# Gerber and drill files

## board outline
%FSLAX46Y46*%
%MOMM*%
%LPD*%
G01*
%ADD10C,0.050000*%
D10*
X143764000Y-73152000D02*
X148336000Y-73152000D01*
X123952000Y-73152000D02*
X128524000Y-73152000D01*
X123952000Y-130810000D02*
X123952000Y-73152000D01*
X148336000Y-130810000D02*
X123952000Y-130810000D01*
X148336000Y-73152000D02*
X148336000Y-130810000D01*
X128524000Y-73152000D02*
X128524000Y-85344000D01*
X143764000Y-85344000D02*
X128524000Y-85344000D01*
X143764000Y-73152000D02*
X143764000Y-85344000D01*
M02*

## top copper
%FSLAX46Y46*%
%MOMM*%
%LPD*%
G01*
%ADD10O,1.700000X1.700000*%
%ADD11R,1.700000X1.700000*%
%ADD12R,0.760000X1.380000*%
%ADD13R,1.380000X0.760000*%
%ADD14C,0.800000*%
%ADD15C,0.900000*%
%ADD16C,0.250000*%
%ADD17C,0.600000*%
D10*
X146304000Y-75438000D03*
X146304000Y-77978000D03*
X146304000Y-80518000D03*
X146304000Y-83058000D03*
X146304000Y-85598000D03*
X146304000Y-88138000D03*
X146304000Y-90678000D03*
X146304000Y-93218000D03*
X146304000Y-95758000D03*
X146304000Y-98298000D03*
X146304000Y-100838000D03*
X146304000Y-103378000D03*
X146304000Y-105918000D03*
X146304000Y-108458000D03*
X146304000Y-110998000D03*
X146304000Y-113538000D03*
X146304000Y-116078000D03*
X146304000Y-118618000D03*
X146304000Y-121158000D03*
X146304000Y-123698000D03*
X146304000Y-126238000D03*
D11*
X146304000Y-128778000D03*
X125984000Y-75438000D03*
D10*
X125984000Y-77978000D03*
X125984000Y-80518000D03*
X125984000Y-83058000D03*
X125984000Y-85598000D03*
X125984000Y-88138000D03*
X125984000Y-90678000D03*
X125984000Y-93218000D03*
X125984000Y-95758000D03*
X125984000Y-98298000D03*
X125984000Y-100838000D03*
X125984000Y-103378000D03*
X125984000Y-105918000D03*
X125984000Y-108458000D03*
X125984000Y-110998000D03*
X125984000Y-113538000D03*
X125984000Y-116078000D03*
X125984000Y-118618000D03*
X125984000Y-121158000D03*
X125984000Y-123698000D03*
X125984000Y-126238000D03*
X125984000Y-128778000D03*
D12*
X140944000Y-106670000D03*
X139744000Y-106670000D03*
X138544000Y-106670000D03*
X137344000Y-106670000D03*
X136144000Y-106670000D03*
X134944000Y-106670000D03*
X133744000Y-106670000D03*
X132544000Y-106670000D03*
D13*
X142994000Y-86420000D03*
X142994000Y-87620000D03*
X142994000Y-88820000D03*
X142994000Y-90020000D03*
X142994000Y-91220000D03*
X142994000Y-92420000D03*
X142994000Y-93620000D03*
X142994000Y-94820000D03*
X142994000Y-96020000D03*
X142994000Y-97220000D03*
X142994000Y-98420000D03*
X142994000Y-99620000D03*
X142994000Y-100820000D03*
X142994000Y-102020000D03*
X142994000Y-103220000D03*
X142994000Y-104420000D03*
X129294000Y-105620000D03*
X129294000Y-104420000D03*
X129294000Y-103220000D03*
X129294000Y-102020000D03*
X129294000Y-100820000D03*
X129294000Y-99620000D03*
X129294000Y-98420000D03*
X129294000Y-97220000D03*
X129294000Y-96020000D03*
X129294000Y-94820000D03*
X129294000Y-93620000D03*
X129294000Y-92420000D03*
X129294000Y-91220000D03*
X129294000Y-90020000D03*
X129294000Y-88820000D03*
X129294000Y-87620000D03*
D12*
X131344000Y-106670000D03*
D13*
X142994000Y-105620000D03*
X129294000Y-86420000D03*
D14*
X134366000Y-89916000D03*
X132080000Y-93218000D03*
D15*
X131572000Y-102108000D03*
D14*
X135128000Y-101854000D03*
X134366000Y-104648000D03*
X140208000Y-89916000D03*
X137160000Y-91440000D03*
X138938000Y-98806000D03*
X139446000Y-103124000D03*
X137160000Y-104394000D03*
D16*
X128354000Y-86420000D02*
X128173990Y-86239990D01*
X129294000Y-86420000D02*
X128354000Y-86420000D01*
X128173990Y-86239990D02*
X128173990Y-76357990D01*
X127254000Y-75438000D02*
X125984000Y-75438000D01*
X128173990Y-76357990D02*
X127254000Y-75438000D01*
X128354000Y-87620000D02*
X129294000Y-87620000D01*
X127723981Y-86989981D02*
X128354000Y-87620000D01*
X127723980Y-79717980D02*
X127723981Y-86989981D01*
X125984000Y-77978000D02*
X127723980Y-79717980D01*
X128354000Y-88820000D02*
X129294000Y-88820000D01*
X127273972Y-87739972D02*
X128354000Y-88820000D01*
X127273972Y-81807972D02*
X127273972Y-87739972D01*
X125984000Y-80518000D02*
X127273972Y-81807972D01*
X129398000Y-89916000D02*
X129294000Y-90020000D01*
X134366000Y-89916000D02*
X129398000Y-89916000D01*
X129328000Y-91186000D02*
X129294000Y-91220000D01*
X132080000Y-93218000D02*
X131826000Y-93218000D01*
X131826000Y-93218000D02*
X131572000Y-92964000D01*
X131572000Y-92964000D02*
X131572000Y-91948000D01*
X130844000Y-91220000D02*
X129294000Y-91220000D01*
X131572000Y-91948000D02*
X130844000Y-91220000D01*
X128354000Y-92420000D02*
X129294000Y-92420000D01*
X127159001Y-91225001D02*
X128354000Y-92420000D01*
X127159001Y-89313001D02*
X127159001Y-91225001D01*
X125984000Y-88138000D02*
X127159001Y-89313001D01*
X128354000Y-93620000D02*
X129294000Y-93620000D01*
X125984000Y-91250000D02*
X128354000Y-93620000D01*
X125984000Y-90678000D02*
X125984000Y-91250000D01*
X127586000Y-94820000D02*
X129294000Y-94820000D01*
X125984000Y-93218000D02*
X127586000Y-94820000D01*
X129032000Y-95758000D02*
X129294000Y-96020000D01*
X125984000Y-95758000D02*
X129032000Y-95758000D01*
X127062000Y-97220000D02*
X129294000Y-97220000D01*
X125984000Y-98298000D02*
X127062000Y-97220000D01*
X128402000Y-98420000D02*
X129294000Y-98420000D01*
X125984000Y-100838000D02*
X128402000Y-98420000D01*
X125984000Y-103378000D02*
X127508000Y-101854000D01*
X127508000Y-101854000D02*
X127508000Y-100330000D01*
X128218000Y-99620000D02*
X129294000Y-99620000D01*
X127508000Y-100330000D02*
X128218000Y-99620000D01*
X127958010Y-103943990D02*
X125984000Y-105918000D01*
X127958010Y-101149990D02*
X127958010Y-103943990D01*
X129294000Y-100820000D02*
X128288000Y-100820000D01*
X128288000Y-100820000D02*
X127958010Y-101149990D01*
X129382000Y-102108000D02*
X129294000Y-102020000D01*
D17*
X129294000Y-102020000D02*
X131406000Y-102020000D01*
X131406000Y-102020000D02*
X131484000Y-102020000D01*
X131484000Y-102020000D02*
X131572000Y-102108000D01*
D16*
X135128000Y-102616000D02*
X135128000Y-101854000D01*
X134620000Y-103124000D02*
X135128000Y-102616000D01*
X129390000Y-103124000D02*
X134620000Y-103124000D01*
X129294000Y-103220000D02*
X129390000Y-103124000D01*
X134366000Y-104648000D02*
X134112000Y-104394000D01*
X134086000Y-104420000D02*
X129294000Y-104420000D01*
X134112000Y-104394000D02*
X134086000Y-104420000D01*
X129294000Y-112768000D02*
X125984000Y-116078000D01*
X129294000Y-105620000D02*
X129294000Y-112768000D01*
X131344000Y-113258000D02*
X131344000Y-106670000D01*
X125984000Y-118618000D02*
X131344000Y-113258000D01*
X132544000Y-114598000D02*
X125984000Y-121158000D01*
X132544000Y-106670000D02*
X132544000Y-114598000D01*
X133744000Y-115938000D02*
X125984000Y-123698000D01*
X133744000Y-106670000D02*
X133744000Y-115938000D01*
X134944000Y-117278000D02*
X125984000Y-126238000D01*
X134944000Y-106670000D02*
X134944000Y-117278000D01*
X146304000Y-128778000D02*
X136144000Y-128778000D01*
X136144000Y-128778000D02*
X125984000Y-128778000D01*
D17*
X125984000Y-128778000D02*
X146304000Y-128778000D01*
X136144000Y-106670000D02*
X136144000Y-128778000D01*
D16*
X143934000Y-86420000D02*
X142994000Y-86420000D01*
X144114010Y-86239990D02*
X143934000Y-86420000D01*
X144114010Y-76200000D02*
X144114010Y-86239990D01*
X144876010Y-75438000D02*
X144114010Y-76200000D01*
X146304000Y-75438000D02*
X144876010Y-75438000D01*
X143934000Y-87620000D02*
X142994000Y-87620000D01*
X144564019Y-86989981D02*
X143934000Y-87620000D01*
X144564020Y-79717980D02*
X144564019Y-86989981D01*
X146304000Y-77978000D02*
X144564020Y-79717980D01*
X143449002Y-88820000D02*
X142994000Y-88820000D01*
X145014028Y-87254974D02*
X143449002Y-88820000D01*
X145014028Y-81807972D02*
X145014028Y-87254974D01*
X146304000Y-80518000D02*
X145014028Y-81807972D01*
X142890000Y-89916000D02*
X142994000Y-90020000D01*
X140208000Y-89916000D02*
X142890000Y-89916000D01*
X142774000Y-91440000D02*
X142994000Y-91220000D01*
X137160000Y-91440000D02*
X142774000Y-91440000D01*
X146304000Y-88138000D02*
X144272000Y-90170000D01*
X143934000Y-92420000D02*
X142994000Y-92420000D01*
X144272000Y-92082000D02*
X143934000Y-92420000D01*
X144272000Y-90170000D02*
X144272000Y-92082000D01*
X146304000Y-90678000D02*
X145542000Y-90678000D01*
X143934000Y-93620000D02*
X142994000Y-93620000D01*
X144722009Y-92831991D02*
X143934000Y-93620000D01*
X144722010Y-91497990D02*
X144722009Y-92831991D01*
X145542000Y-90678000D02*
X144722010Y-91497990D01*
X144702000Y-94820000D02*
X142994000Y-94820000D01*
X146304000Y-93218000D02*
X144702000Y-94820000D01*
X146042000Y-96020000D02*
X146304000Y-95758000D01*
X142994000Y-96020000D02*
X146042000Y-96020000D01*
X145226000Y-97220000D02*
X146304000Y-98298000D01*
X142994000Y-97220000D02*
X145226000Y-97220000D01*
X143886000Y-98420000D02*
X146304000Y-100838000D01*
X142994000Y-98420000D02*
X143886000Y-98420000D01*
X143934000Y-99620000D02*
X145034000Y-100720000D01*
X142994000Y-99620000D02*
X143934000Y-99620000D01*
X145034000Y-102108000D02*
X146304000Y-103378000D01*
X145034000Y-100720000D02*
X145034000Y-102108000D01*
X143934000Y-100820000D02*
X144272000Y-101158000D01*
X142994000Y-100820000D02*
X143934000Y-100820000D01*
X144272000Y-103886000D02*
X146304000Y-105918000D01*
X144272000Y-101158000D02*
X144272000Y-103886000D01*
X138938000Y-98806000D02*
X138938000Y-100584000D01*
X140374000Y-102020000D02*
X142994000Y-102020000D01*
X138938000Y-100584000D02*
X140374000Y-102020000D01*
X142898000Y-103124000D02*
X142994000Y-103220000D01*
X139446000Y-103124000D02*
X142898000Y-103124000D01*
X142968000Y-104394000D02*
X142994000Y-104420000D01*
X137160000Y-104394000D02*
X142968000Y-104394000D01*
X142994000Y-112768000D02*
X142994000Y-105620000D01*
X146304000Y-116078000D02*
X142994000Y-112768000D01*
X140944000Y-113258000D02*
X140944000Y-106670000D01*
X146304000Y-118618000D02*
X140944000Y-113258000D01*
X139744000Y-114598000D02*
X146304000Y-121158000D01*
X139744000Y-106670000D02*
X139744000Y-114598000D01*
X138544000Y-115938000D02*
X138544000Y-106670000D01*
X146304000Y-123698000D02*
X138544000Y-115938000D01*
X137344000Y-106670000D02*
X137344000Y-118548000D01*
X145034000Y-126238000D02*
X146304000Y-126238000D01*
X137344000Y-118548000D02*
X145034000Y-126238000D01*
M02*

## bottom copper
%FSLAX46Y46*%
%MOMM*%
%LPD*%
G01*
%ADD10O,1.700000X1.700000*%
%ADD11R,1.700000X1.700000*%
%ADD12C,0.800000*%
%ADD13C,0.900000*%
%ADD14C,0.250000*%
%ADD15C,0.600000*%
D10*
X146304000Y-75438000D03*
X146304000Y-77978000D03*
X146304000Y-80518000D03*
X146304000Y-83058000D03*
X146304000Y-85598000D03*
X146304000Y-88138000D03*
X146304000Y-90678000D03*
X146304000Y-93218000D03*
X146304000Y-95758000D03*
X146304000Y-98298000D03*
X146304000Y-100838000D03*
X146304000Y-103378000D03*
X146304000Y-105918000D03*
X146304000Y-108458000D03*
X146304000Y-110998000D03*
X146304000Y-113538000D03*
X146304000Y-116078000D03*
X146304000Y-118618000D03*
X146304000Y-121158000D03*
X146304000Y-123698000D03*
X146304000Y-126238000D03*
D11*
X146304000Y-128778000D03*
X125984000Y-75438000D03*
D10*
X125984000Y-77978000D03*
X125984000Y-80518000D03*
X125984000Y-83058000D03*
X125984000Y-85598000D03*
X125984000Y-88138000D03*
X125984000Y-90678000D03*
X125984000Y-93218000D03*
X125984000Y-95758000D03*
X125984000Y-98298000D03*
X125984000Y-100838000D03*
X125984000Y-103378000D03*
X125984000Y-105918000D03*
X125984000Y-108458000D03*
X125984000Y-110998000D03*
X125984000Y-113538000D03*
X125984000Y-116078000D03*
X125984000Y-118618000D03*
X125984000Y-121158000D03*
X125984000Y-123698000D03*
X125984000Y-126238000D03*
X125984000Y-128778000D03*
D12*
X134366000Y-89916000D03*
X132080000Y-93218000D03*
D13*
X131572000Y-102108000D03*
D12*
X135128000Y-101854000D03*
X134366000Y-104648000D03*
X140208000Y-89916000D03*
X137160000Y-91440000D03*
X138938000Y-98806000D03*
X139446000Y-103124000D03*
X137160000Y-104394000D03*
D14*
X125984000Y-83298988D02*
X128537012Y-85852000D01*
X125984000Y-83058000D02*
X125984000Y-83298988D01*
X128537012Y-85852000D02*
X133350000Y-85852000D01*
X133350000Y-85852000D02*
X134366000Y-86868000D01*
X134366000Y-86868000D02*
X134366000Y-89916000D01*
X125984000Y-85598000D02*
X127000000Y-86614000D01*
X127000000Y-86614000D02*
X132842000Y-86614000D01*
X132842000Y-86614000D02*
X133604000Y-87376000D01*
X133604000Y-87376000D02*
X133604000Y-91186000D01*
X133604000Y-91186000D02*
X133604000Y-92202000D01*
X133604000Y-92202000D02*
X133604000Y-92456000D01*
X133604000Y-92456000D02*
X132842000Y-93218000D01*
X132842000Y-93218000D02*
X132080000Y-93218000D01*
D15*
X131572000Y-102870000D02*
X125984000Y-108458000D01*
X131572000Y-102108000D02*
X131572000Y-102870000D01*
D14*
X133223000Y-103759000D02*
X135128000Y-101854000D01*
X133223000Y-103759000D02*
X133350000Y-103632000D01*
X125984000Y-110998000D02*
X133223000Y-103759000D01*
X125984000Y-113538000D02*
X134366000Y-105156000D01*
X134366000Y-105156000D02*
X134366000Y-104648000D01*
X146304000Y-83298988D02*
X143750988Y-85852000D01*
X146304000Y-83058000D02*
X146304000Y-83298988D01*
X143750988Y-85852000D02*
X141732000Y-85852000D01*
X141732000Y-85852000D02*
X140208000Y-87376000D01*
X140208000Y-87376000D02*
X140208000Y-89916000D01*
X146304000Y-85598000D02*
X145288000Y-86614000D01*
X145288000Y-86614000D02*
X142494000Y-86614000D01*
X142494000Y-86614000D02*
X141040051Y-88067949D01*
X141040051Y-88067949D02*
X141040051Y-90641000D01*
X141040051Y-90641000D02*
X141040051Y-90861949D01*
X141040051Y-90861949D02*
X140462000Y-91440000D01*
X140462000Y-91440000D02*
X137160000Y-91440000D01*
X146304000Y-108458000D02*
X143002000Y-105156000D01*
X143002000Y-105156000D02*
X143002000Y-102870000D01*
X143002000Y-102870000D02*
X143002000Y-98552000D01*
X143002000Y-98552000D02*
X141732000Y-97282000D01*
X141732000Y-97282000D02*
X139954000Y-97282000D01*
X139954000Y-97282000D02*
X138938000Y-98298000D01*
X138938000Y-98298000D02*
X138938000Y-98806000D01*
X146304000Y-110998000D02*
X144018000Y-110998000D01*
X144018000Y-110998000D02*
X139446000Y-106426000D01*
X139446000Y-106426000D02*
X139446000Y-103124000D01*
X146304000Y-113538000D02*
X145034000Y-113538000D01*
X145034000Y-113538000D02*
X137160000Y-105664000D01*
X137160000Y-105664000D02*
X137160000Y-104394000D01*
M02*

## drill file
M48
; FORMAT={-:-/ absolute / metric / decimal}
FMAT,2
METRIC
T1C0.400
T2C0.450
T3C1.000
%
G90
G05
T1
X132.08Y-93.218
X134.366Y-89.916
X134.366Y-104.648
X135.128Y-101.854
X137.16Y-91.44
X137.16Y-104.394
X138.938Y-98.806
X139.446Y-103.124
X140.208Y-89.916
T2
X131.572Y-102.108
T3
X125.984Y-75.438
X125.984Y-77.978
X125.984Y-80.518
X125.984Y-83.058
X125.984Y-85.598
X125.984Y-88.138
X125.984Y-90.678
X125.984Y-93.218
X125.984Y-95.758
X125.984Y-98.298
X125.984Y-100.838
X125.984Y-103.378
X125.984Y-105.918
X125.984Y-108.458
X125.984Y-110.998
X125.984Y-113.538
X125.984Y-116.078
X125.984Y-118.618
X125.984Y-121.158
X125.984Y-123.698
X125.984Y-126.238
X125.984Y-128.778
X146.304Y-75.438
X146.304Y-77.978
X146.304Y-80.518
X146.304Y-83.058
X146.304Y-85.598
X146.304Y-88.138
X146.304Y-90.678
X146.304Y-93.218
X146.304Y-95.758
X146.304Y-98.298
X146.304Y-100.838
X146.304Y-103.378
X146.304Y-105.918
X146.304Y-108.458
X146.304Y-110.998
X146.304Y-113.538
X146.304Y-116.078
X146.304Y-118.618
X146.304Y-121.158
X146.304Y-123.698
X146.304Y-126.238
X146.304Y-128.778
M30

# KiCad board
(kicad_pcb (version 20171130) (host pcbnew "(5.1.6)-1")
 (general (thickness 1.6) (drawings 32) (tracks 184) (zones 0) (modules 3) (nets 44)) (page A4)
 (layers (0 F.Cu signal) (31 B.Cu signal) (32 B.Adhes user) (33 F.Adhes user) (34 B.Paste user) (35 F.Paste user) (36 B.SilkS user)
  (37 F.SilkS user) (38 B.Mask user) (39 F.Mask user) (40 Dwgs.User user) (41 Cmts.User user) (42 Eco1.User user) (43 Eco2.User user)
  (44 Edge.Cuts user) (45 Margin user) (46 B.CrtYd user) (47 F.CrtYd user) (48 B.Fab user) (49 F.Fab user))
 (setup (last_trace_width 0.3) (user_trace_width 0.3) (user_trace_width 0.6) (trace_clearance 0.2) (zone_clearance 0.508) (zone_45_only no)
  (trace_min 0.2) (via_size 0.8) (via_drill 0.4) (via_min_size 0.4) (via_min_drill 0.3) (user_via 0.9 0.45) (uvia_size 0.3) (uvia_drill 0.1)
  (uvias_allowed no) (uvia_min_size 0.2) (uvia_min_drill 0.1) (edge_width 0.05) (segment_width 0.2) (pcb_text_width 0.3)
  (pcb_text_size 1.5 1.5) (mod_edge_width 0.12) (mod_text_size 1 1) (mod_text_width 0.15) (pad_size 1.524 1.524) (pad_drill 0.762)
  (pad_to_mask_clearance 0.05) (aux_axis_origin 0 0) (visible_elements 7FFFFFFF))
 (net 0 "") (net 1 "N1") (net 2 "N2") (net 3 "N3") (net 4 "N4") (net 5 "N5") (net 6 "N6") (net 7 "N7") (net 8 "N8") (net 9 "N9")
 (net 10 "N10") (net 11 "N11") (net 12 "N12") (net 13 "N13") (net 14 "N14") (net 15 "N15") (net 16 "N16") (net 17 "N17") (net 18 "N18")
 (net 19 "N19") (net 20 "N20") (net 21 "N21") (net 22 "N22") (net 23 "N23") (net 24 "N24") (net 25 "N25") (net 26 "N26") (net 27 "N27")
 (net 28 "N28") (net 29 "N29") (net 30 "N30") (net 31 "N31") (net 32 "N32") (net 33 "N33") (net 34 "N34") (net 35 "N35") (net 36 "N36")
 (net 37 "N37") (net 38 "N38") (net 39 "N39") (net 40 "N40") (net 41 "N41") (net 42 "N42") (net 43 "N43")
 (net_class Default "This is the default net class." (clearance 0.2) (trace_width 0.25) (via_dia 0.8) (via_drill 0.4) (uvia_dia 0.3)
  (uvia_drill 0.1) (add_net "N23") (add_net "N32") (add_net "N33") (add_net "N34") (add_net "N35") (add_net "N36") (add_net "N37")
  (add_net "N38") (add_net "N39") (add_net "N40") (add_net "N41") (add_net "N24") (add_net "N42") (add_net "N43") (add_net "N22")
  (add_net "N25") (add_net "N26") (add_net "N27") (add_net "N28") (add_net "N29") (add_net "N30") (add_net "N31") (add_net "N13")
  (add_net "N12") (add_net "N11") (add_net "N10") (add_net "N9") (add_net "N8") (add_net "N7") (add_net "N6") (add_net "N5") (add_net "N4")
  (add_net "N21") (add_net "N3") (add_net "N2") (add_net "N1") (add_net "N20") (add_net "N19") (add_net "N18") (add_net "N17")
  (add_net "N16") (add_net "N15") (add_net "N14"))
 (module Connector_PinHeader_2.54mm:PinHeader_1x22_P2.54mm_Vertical (layer F.Cu) (at 146.304 128.778 180)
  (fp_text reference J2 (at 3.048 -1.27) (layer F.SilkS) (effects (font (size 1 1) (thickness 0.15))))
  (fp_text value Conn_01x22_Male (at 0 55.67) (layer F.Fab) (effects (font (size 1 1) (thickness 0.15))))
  (pad 22 thru_hole oval (at 0 53.34 180) (size 1.7 1.7) (drill 1) (layers *.Cu *.Mask) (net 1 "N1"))
  (pad 21 thru_hole oval (at 0 50.8 180) (size 1.7 1.7) (drill 1) (layers *.Cu *.Mask) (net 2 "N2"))
  (pad 20 thru_hole oval (at 0 48.26 180) (size 1.7 1.7) (drill 1) (layers *.Cu *.Mask) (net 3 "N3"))
  (pad 19 thru_hole oval (at 0 45.72 180) (size 1.7 1.7) (drill 1) (layers *.Cu *.Mask) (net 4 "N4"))
  (pad 18 thru_hole oval (at 0 43.18 180) (size 1.7 1.7) (drill 1) (layers *.Cu *.Mask) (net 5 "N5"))
  (pad 17 thru_hole oval (at 0 40.64 180) (size 1.7 1.7) (drill 1) (layers *.Cu *.Mask) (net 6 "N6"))
  (pad 16 thru_hole oval (at 0 38.1 180) (size 1.7 1.7) (drill 1) (layers *.Cu *.Mask) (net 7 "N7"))
  (pad 15 thru_hole oval (at 0 35.56 180) (size 1.7 1.7) (drill 1) (layers *.Cu *.Mask) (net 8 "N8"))
  (pad 14 thru_hole oval (at 0 33.02 180) (size 1.7 1.7) (drill 1) (layers *.Cu *.Mask) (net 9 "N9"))
  (pad 13 thru_hole oval (at 0 30.48 180) (size 1.7 1.7) (drill 1) (layers *.Cu *.Mask) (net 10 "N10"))
  (pad 12 thru_hole oval (at 0 27.94 180) (size 1.7 1.7) (drill 1) (layers *.Cu *.Mask) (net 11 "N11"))
  (pad 11 thru_hole oval (at 0 25.4 180) (size 1.7 1.7) (drill 1) (layers *.Cu *.Mask) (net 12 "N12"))
  (pad 10 thru_hole oval (at 0 22.86 180) (size 1.7 1.7) (drill 1) (layers *.Cu *.Mask) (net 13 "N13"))
  (pad 9 thru_hole oval (at 0 20.32 180) (size 1.7 1.7) (drill 1) (layers *.Cu *.Mask) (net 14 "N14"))
  (pad 8 thru_hole oval (at 0 17.78 180) (size 1.7 1.7) (drill 1) (layers *.Cu *.Mask) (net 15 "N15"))
  (pad 7 thru_hole oval (at 0 15.24 180) (size 1.7 1.7) (drill 1) (layers *.Cu *.Mask) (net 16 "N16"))
  (pad 6 thru_hole oval (at 0 12.7 180) (size 1.7 1.7) (drill 1) (layers *.Cu *.Mask) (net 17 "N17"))
  (pad 5 thru_hole oval (at 0 10.16 180) (size 1.7 1.7) (drill 1) (layers *.Cu *.Mask) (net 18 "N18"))
  (pad 4 thru_hole oval (at 0 7.62 180) (size 1.7 1.7) (drill 1) (layers *.Cu *.Mask) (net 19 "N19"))
  (pad 3 thru_hole oval (at 0 5.08 180) (size 1.7 1.7) (drill 1) (layers *.Cu *.Mask) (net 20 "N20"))
  (pad 2 thru_hole oval (at 0 2.54 180) (size 1.7 1.7) (drill 1) (layers *.Cu *.Mask) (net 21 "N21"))
  (pad 1 thru_hole rect (at 0 0 180) (size 1.7 1.7) (drill 1) (layers *.Cu *.Mask) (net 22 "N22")))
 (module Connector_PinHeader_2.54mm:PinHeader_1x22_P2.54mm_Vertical (layer F.Cu) (at 125.984 75.438)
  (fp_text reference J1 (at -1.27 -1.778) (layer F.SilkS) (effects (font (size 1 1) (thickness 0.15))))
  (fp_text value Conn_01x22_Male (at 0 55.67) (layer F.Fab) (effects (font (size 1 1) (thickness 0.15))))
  (pad 1 thru_hole rect (at 0 0) (size 1.7 1.7) (drill 1) (layers *.Cu *.Mask) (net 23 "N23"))
  (pad 2 thru_hole oval (at 0 2.54) (size 1.7 1.7) (drill 1) (layers *.Cu *.Mask) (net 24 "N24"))
  (pad 3 thru_hole oval (at 0 5.08) (size 1.7 1.7) (drill 1) (layers *.Cu *.Mask) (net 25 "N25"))
  (pad 4 thru_hole oval (at 0 7.62) (size 1.7 1.7) (drill 1) (layers *.Cu *.Mask) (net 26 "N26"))
  (pad 5 thru_hole oval (at 0 10.16) (size 1.7 1.7) (drill 1) (layers *.Cu *.Mask) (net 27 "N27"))
  (pad 6 thru_hole oval (at 0 12.7) (size 1.7 1.7) (drill 1) (layers *.Cu *.Mask) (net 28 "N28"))
  (pad 7 thru_hole oval (at 0 15.24) (size 1.7 1.7) (drill 1) (layers *.Cu *.Mask) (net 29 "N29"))
  (pad 8 thru_hole oval (at 0 17.78) (size 1.7 1.7) (drill 1) (layers *.Cu *.Mask) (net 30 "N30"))
  (pad 9 thru_hole oval (at 0 20.32) (size 1.7 1.7) (drill 1) (layers *.Cu *.Mask) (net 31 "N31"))
  (pad 10 thru_hole oval (at 0 22.86) (size 1.7 1.7) (drill 1) (layers *.Cu *.Mask) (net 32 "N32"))
  (pad 11 thru_hole oval (at 0 25.4) (size 1.7 1.7) (drill 1) (layers *.Cu *.Mask) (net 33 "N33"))
  (pad 12 thru_hole oval (at 0 27.94) (size 1.7 1.7) (drill 1) (layers *.Cu *.Mask) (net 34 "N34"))
  (pad 13 thru_hole oval (at 0 30.48) (size 1.7 1.7) (drill 1) (layers *.Cu *.Mask) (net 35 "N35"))
  (pad 14 thru_hole oval (at 0 33.02) (size 1.7 1.7) (drill 1) (layers *.Cu *.Mask) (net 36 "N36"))
  (pad 15 thru_hole oval (at 0 35.56) (size 1.7 1.7) (drill 1) (layers *.Cu *.Mask) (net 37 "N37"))
  (pad 16 thru_hole oval (at 0 38.1) (size 1.7 1.7) (drill 1) (layers *.Cu *.Mask) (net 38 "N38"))
  (pad 17 thru_hole oval (at 0 40.64) (size 1.7 1.7) (drill 1) (layers *.Cu *.Mask) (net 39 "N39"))
  (pad 18 thru_hole oval (at 0 43.18) (size 1.7 1.7) (drill 1) (layers *.Cu *.Mask) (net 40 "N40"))
  (pad 19 thru_hole oval (at 0 45.72) (size 1.7 1.7) (drill 1) (layers *.Cu *.Mask) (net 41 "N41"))
  (pad 20 thru_hole oval (at 0 48.26) (size 1.7 1.7) (drill 1) (layers *.Cu *.Mask) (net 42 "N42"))
  (pad 21 thru_hole oval (at 0 50.8) (size 1.7 1.7) (drill 1) (layers *.Cu *.Mask) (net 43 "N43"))
  (pad 22 thru_hole oval (at 0 53.34) (size 1.7 1.7) (drill 1) (layers *.Cu *.Mask) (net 22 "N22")))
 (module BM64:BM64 (layer F.Cu) (at 136.144 83.82)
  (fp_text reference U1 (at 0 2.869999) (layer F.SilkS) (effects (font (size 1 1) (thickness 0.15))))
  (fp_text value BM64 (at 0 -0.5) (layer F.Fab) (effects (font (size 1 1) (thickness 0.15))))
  (pad 26 smd rect (at 4.8 22.85 90) (size 1.38 0.76) (layers F.Cu F.Paste F.Mask) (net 18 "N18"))
  (pad 25 smd rect (at 3.6 22.85 90) (size 1.38 0.76) (layers F.Cu F.Paste F.Mask) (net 19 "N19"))
  (pad 24 smd rect (at 2.4 22.85 90) (size 1.38 0.76) (layers F.Cu F.Paste F.Mask) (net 20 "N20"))
  (pad 23 smd rect (at 1.2 22.85 90) (size 1.38 0.76) (layers F.Cu F.Paste F.Mask) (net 21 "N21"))
  (pad 22 smd rect (at 0 22.85 90) (size 1.38 0.76) (layers F.Cu F.Paste F.Mask) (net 22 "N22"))
  (pad 21 smd rect (at -1.2 22.85 90) (size 1.38 0.76) (layers F.Cu F.Paste F.Mask) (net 43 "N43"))
  (pad 20 smd rect (at -2.4 22.85 90) (size 1.38 0.76) (layers F.Cu F.Paste F.Mask) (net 42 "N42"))
  (pad 19 smd rect (at -3.6 22.85 90) (size 1.38 0.76) (layers F.Cu F.Paste F.Mask) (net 41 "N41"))
  (pad 43 smd rect (at 6.85 2.6) (size 1.38 0.76) (layers F.Cu F.Paste F.Mask) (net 1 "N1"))
  (pad 42 smd rect (at 6.85 3.8) (size 1.38 0.76) (layers F.Cu F.Paste F.Mask) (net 2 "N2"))
  (pad 41 smd rect (at 6.85 5) (size 1.38 0.76) (layers F.Cu F.Paste F.Mask) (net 3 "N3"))
  (pad 40 smd rect (at 6.85 6.2) (size 1.38 0.76) (layers F.Cu F.Paste F.Mask) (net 4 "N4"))
  (pad 39 smd rect (at 6.85 7.4) (size 1.38 0.76) (layers F.Cu F.Paste F.Mask) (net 5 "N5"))
  (pad 38 smd rect (at 6.85 8.6) (size 1.38 0.76) (layers F.Cu F.Paste F.Mask) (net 6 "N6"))
  (pad 37 smd rect (at 6.85 9.8) (size 1.38 0.76) (layers F.Cu F.Paste F.Mask) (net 7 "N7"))
  (pad 36 smd rect (at 6.85 11) (size 1.38 0.76) (layers F.Cu F.Paste F.Mask) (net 8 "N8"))
  (pad 35 smd rect (at 6.85 12.2) (size 1.38 0.76) (layers F.Cu F.Paste F.Mask) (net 9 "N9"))
  (pad 34 smd rect (at 6.85 13.4) (size 1.38 0.76) (layers F.Cu F.Paste F.Mask) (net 10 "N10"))
  (pad 33 smd rect (at 6.85 14.6) (size 1.38 0.76) (layers F.Cu F.Paste F.Mask) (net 11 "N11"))
  (pad 32 smd rect (at 6.85 15.8) (size 1.38 0.76) (layers F.Cu F.Paste F.Mask) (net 12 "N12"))
  (pad 31 smd rect (at 6.85 17) (size 1.38 0.76) (layers F.Cu F.Paste F.Mask) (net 13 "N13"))
  (pad 30 smd rect (at 6.85 18.2) (size 1.38 0.76) (layers F.Cu F.Paste F.Mask) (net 14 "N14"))
  (pad 29 smd rect (at 6.85 19.4) (size 1.38 0.76) (layers F.Cu F.Paste F.Mask) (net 15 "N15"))
  (pad 28 smd rect (at 6.85 20.6) (size 1.38 0.76) (layers F.Cu F.Paste F.Mask) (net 16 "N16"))
  (pad 17 smd rect (at -6.85 21.8) (size 1.38 0.76) (layers F.Cu F.Paste F.Mask) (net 39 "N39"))
  (pad 16 smd rect (at -6.85 20.6) (size 1.38 0.76) (layers F.Cu F.Paste F.Mask) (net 38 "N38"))
  (pad 15 smd rect (at -6.85 19.4) (size 1.38 0.76) (layers F.Cu F.Paste F.Mask) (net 37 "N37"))
  (pad 14 smd rect (at -6.85 18.2) (size 1.38 0.76) (layers F.Cu F.Paste F.Mask) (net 36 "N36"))
  (pad 13 smd rect (at -6.85 17) (size 1.38 0.76) (layers F.Cu F.Paste F.Mask) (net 35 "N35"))
  (pad 12 smd rect (at -6.85 15.8) (size 1.38 0.76) (layers F.Cu F.Paste F.Mask) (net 34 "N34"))
  (pad 11 smd rect (at -6.85 14.6) (size 1.38 0.76) (layers F.Cu F.Paste F.Mask) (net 33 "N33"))
  (pad 10 smd rect (at -6.85 13.4) (size 1.38 0.76) (layers F.Cu F.Paste F.Mask) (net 32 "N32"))
  (pad 9 smd rect (at -6.85 12.2) (size 1.38 0.76) (layers F.Cu F.Paste F.Mask) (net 31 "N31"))
  (pad 8 smd rect (at -6.85 11) (size 1.38 0.76) (layers F.Cu F.Paste F.Mask) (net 30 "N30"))
  (pad 7 smd rect (at -6.85 9.8) (size 1.38 0.76) (layers F.Cu F.Paste F.Mask) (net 29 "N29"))
  (pad 6 smd rect (at -6.85 8.6) (size 1.38 0.76) (layers F.Cu F.Paste F.Mask) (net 28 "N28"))
  (pad 5 smd rect (at -6.85 7.4) (size 1.38 0.76) (layers F.Cu F.Paste F.Mask) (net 27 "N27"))
  (pad 4 smd rect (at -6.85 6.2) (size 1.38 0.76) (layers F.Cu F.Paste F.Mask) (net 26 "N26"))
  (pad 3 smd rect (at -6.85 5) (size 1.38 0.76) (layers F.Cu F.Paste F.Mask) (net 25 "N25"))
  (pad 2 smd rect (at -6.85 3.8) (size 1.38 0.76) (layers F.Cu F.Paste F.Mask) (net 24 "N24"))
  (pad 18 smd rect (at -4.8 22.85 90) (size 1.38 0.76) (layers F.Cu F.Paste F.Mask) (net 40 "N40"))
  (pad 27 smd rect (at 6.85 21.8) (size 1.38 0.76) (layers F.Cu F.Paste F.Mask) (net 17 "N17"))
  (pad 1 smd rect (at -6.85 2.6) (size 1.38 0.76) (layers F.Cu F.Paste F.Mask) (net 23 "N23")))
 (gr_line (start 143.764 73.152) (end 148.336 73.152) (layer Edge.Cuts) (width 0.05))
 (gr_line (start 123.952 73.152) (end 128.524 73.152) (layer Edge.Cuts) (width 0.05))
 (gr_line (start 123.952 130.81) (end 123.952 73.152) (layer Edge.Cuts) (width 0.05))
 (gr_line (start 148.336 130.81) (end 123.952 130.81) (layer Edge.Cuts) (width 0.05))
 (gr_line (start 148.336 73.152) (end 148.336 130.81) (layer Edge.Cuts) (width 0.05))
 (gr_line (start 128.524 73.152) (end 128.524 85.344) (layer Edge.Cuts) (width 0.05))
 (gr_line (start 143.764 85.344) (end 128.524 85.344) (layer Edge.Cuts) (width 0.05))
 (gr_line (start 143.764 73.152) (end 143.764 85.344) (layer Edge.Cuts) (width 0.05))
 (segment (start 128.354 86.42) (end 128.17399 86.23999) (width 0.25) (layer F.Cu) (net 23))
 (segment (start 129.294 86.42) (end 128.354 86.42) (width 0.25) (layer F.Cu) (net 23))
 (segment (start 128.17399 86.23999) (end 128.17399 76.35799) (width 0.25) (layer F.Cu) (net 23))
 (segment (start 127.254 75.438) (end 125.984 75.438) (width 0.25) (layer F.Cu) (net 23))
 (segment (start 128.17399 76.35799) (end 127.254 75.438) (width 0.25) (layer F.Cu) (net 23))
 (segment (start 128.354 87.62) (end 129.294 87.62) (width 0.25) (layer F.Cu) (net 24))
 (segment (start 127.723981 86.989981) (end 128.354 87.62) (width 0.25) (layer F.Cu) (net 24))
 (segment (start 127.72398 79.71798) (end 127.723981 86.989981) (width 0.25) (layer F.Cu) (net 24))
 (segment (start 125.984 77.978) (end 127.72398 79.71798) (width 0.25) (layer F.Cu) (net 24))
 (segment (start 128.354 88.82) (end 129.294 88.82) (width 0.25) (layer F.Cu) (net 25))
 (segment (start 127.273972 87.739972) (end 128.354 88.82) (width 0.25) (layer F.Cu) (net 25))
 (segment (start 127.273972 81.807972) (end 127.273972 87.739972) (width 0.25) (layer F.Cu) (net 25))
 (segment (start 125.984 80.518) (end 127.273972 81.807972) (width 0.25) (layer F.Cu) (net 25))
 (segment (start 125.984 83.298988) (end 128.537012 85.852) (width 0.25) (layer B.Cu) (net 26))
 (segment (start 125.984 83.058) (end 125.984 83.298988) (width 0.25) (layer B.Cu) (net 26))
 (segment (start 128.537012 85.852) (end 133.35 85.852) (width 0.25) (layer B.Cu) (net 26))
 (via (at 134.366 89.916) (size 0.8) (drill 0.4) (layers F.Cu B.Cu) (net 26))
 (segment (start 133.35 85.852) (end 134.366 86.868) (width 0.25) (layer B.Cu) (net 26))
 (segment (start 134.366 86.868) (end 134.366 89.916) (width 0.25) (layer B.Cu) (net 26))
 (segment (start 129.398 89.916) (end 129.294 90.02) (width 0.25) (layer F.Cu) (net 26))
 (segment (start 134.366 89.916) (end 129.398 89.916) (width 0.25) (layer F.Cu) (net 26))
 (segment (start 125.984 85.598) (end 127 86.614) (width 0.25) (layer B.Cu) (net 27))
 (segment (start 127 86.614) (end 132.842 86.614) (width 0.25) (layer B.Cu) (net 27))
 (segment (start 132.842 86.614) (end 133.604 87.376) (width 0.25) (layer B.Cu) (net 27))
 (segment (start 133.604 87.376) (end 133.604 91.186) (width 0.25) (layer B.Cu) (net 27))
 (segment (start 129.328 91.186) (end 129.294 91.22) (width 0.25) (layer F.Cu) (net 27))
 (segment (start 133.604 91.186) (end 133.604 92.202) (width 0.25) (layer B.Cu) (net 27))
 (segment (start 133.604 92.202) (end 133.604 92.456) (width 0.25) (layer B.Cu) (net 27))
 (via (at 132.08 93.218) (size 0.8) (drill 0.4) (layers F.Cu B.Cu) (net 27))
 (segment (start 133.604 92.456) (end 132.842 93.218) (width 0.25) (layer B.Cu) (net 27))
 (segment (start 132.842 93.218) (end 132.08 93.218) (width 0.25) (layer B.Cu) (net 27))
 (segment (start 132.08 93.218) (end 131.826 93.218) (width 0.25) (layer F.Cu) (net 27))
 (segment (start 131.826 93.218) (end 131.572 92.964) (width 0.25) (layer F.Cu) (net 27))
 (segment (start 131.572 92.964) (end 131.572 91.948) (width 0.25) (layer F.Cu) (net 27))
 (segment (start 130.844 91.22) (end 129.294 91.22) (width 0.25) (layer F.Cu) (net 27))
 (segment (start 131.572 91.948) (end 130.844 91.22) (width 0.25) (layer F.Cu) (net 27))
 (segment (start 128.354 92.42) (end 129.294 92.42) (width 0.25) (layer F.Cu) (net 28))
 (segment (start 127.159001 91.225001) (end 128.354 92.42) (width 0.25) (layer F.Cu) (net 28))
 (segment (start 127.159001 89.313001) (end 127.159001 91.225001) (width 0.25) (layer F.Cu) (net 28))
 (segment (start 125.984 88.138) (end 127.159001 89.313001) (width 0.25) (layer F.Cu) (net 28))
 (segment (start 128.354 93.62) (end 129.294 93.62) (width 0.25) (layer F.Cu) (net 29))
 (segment (start 125.984 91.25) (end 128.354 93.62) (width 0.25) (layer F.Cu) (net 29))
 (segment (start 125.984 90.678) (end 125.984 91.25) (width 0.25) (layer F.Cu) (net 29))
 (segment (start 127.586 94.82) (end 129.294 94.82) (width 0.25) (layer F.Cu) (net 30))
 (segment (start 125.984 93.218) (end 127.586 94.82) (width 0.25) (layer F.Cu) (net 30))
 (segment (start 129.032 95.758) (end 129.294 96.02) (width 0.25) (layer F.Cu) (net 31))
 (segment (start 125.984 95.758) (end 129.032 95.758) (width 0.25) (layer F.Cu) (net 31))
 (segment (start 127.062 97.22) (end 129.294 97.22) (width 0.25) (layer F.Cu) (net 32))
 (segment (start 125.984 98.298) (end 127.062 97.22) (width 0.25) (layer F.Cu) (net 32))
 (segment (start 128.402 98.42) (end 129.294 98.42) (width 0.25) (layer F.Cu) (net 33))
 (segment (start 125.984 100.838) (end 128.402 98.42) (width 0.25) (layer F.Cu) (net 33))
 (segment (start 125.984 103.378) (end 127.508 101.854) (width 0.25) (layer F.Cu) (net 34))
 (segment (start 127.508 101.854) (end 127.508 100.33) (width 0.25) (layer F.Cu) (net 34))
 (segment (start 128.218 99.62) (end 129.294 99.62) (width 0.25) (layer F.Cu) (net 34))
 (segment (start 127.508 100.33) (end 128.218 99.62) (width 0.25) (layer F.Cu) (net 34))
 (segment (start 127.95801 103.94399) (end 125.984 105.918) (width 0.25) (layer F.Cu) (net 35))
 (segment (start 127.95801 101.14999) (end 127.95801 103.94399) (width 0.25) (layer F.Cu) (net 35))
 (segment (start 129.294 100.82) (end 128.288 100.82) (width 0.25) (layer F.Cu) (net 35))
 (segment (start 128.288 100.82) (end 127.95801 101.14999) (width 0.25) (layer F.Cu) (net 35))
 (segment (start 129.382 102.108) (end 129.294 102.02) (width 0.25) (layer F.Cu) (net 36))
 (segment (start 129.294 102.02) (end 131.406 102.02) (width 0.6) (layer F.Cu) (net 36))
 (segment (start 131.572 102.87) (end 125.984 108.458) (width 0.6) (layer B.Cu) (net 36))
 (via (at 131.572 102.108) (size 0.9) (drill 0.45) (layers F.Cu B.Cu) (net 36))
 (segment (start 131.406 102.02) (end 131.484 102.02) (width 0.6) (layer F.Cu) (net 36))
 (segment (start 131.484 102.02) (end 131.572 102.108) (width 0.6) (layer F.Cu) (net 36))
 (segment (start 131.572 102.108) (end 131.572 102.87) (width 0.6) (layer B.Cu) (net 36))
 (via (at 135.128 101.854) (size 0.8) (drill 0.4) (layers F.Cu B.Cu) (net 37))
 (segment (start 133.223 103.759) (end 135.128 101.854) (width 0.25) (layer B.Cu) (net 37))
 (segment (start 133.223 103.759) (end 133.35 103.632) (width 0.25) (layer B.Cu) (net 37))
 (segment (start 125.984 110.998) (end 133.223 103.759) (width 0.25) (layer B.Cu) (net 37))
 (segment (start 135.128 102.616) (end 135.128 101.854) (width 0.25) (layer F.Cu) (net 37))
 (segment (start 134.62 103.124) (end 135.128 102.616) (width 0.25) (layer F.Cu) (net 37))
 (segment (start 129.39 103.124) (end 134.62 103.124) (width 0.25) (layer F.Cu) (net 37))
 (segment (start 129.294 103.22) (end 129.39 103.124) (width 0.25) (layer F.Cu) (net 37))
 (segment (start 125.984 113.538) (end 134.366 105.156) (width 0.25) (layer B.Cu) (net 38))
 (via (at 134.366 104.648) (size 0.8) (drill 0.4) (layers F.Cu B.Cu) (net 38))
 (segment (start 134.366 105.156) (end 134.366 104.648) (width 0.25) (layer B.Cu) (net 38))
 (segment (start 134.366 104.648) (end 134.112 104.394) (width 0.25) (layer F.Cu) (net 38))
 (segment (start 134.086 104.42) (end 129.294 104.42) (width 0.25) (layer F.Cu) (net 38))
 (segment (start 134.112 104.394) (end 134.086 104.42) (width 0.25) (layer F.Cu) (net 38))
 (segment (start 129.294 112.768) (end 125.984 116.078) (width 0.25) (layer F.Cu) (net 39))
 (segment (start 129.294 105.62) (end 129.294 112.768) (width 0.25) (layer F.Cu) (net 39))
 (segment (start 131.344 113.258) (end 131.344 106.67) (width 0.25) (layer F.Cu) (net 40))
 (segment (start 125.984 118.618) (end 131.344 113.258) (width 0.25) (layer F.Cu) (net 40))
 (segment (start 132.544 114.598) (end 125.984 121.158) (width 0.25) (layer F.Cu) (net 41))
 (segment (start 132.544 106.67) (end 132.544 114.598) (width 0.25) (layer F.Cu) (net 41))
 (segment (start 133.744 115.938) (end 125.984 123.698) (width 0.25) (layer F.Cu) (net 42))
 (segment (start 133.744 106.67) (end 133.744 115.938) (width 0.25) (layer F.Cu) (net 42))
 (segment (start 134.944 117.278) (end 125.984 126.238) (width 0.25) (layer F.Cu) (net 43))
 (segment (start 134.944 106.67) (end 134.944 117.278) (width 0.25) (layer F.Cu) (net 43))
 (segment (start 146.304 128.778) (end 136.144 128.778) (width 0.25) (layer F.Cu) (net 22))
 (segment (start 136.144 128.778) (end 125.984 128.778) (width 0.25) (layer F.Cu) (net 22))
 (segment (start 125.984 128.778) (end 146.304 128.778) (width 0.6) (layer F.Cu) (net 22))
 (segment (start 136.144 106.67) (end 136.144 128.778) (width 0.6) (layer F.Cu) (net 22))
 (segment (start 143.934 86.42) (end 142.994 86.42) (width 0.25) (layer F.Cu) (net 1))
 (segment (start 144.11401 86.23999) (end 143.934 86.42) (width 0.25) (layer F.Cu) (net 1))
 (segment (start 144.11401 76.2) (end 144.11401 86.23999) (width 0.25) (layer F.Cu) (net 1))
 (segment (start 144.87601 75.438) (end 144.11401 76.2) (width 0.25) (layer F.Cu) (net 1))
 (segment (start 146.304 75.438) (end 144.87601 75.438) (width 0.25) (layer F.Cu) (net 1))
 (segment (start 143.934 87.62) (end 142.994 87.62) (width 0.25) (layer F.Cu) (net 2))
 (segment (start 144.564019 86.989981) (end 143.934 87.62) (width 0.25) (layer F.Cu) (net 2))
 (segment (start 144.56402 79.71798) (end 144.564019 86.989981) (width 0.25) (layer F.Cu) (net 2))
 (segment (start 146.304 77.978) (end 144.56402 79.71798) (width 0.25) (layer F.Cu) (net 2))
 (segment (start 143.449002 88.82) (end 142.994 88.82) (width 0.25) (layer F.Cu) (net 3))
 (segment (start 145.014028 87.254974) (end 143.449002 88.82) (width 0.25) (layer F.Cu) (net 3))
 (segment (start 145.014028 81.807972) (end 145.014028 87.254974) (width 0.25) (layer F.Cu) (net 3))
 (segment (start 146.304 80.518) (end 145.014028 81.807972) (width 0.25) (layer F.Cu) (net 3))
 (segment (start 146.304 83.298988) (end 143.750988 85.852) (width 0.25) (layer B.Cu) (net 4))
 (segment (start 146.304 83.058) (end 146.304 83.298988) (width 0.25) (layer B.Cu) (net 4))
 (segment (start 143.750988 85.852) (end 141.732 85.852) (width 0.25) (layer B.Cu) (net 4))
 (via (at 140.208 89.916) (size 0.8) (drill 0.4) (layers F.Cu B.Cu) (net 4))
 (segment (start 141.732 85.852) (end 140.208 87.376) (width 0.25) (layer B.Cu) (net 4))
 (segment (start 140.208 87.376) (end 140.208 89.916) (width 0.25) (layer B.Cu) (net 4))
 (segment (start 142.89 89.916) (end 142.994 90.02) (width 0.25) (layer F.Cu) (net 4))
 (segment (start 140.208 89.916) (end 142.89 89.916) (width 0.25) (layer F.Cu) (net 4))
 (segment (start 146.304 85.598) (end 145.288 86.614) (width 0.25) (layer B.Cu) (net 5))
 (segment (start 145.288 86.614) (end 142.494 86.614) (width 0.25) (layer B.Cu) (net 5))
 (segment (start 142.494 86.614) (end 141.040051 88.067949) (width 0.25) (layer B.Cu) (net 5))
 (segment (start 141.040051 88.067949) (end 141.040051 90.641) (width 0.25) (layer B.Cu) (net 5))
 (segment (start 141.040051 90.641) (end 141.040051 90.861949) (width 0.25) (layer B.Cu) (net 5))
 (via (at 137.16 91.44) (size 0.8) (drill 0.4) (layers F.Cu B.Cu) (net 5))
 (segment (start 141.040051 90.861949) (end 140.462 91.44) (width 0.25) (layer B.Cu) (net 5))
 (segment (start 140.462 91.44) (end 137.16 91.44) (width 0.25) (layer B.Cu) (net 5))
 (segment (start 142.774 91.44) (end 142.994 91.22) (width 0.25) (layer F.Cu) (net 5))
 (segment (start 137.16 91.44) (end 142.774 91.44) (width 0.25) (layer F.Cu) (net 5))
 (segment (start 146.304 88.138) (end 144.272 90.17) (width 0.25) (layer F.Cu) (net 6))
 (segment (start 143.934 92.42) (end 142.994 92.42) (width 0.25) (layer F.Cu) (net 6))
 (segment (start 144.272 92.082) (end 143.934 92.42) (width 0.25) (layer F.Cu) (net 6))
 (segment (start 144.272 90.17) (end 144.272 92.082) (width 0.25) (layer F.Cu) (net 6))
 (segment (start 146.304 90.678) (end 145.542 90.678) (width 0.25) (layer F.Cu) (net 7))
 (segment (start 143.934 93.62) (end 142.994 93.62) (width 0.25) (layer F.Cu) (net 7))
 (segment (start 144.722009 92.831991) (end 143.934 93.62) (width 0.25) (layer F.Cu) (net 7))
 (segment (start 144.72201 91.49799) (end 144.722009 92.831991) (width 0.25) (layer F.Cu) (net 7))
 (segment (start 145.542 90.678) (end 144.72201 91.49799) (width 0.25) (layer F.Cu) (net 7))
 (segment (start 144.702 94.82) (end 142.994 94.82) (width 0.25) (layer F.Cu) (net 8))
 (segment (start 146.304 93.218) (end 144.702 94.82) (width 0.25) (layer F.Cu) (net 8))
 (segment (start 146.042 96.02) (end 146.304 95.758) (width 0.25) (layer F.Cu) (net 9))
 (segment (start 142.994 96.02) (end 146.042 96.02) (width 0.25) (layer F.Cu) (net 9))
 (segment (start 145.226 97.22) (end 146.304 98.298) (width 0.25) (layer F.Cu) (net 10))
 (segment (start 142.994 97.22) (end 145.226 97.22) (width 0.25) (layer F.Cu) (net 10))
 (segment (start 143.886 98.42) (end 146.304 100.838) (width 0.25) (layer F.Cu) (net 11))
 (segment (start 142.994 98.42) (end 143.886 98.42) (width 0.25) (layer F.Cu) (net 11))
 (segment (start 143.934 99.62) (end 145.034 100.72) (width 0.25) (layer F.Cu) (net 12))
 (segment (start 142.994 99.62) (end 143.934 99.62) (width 0.25) (layer F.Cu) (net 12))
 (segment (start 145.034 102.108) (end 146.304 103.378) (width 0.25) (layer F.Cu) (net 12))
 (segment (start 145.034 100.72) (end 145.034 102.108) (width 0.25) (layer F.Cu) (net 12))
 (segment (start 143.934 100.82) (end 144.272 101.158) (width 0.25) (layer F.Cu) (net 13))
 (segment (start 142.994 100.82) (end 143.934 100.82) (width 0.25) (layer F.Cu) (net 13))
 (segment (start 144.272 103.886) (end 146.304 105.918) (width 0.25) (layer F.Cu) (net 13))
 (segment (start 144.272 101.158) (end 144.272 103.886) (width 0.25) (layer F.Cu) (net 13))
 (segment (start 146.304 108.458) (end 143.002 105.156) (width 0.25) (layer B.Cu) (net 14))
 (segment (start 143.002 105.156) (end 143.002 102.87) (width 0.25) (layer B.Cu) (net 14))
 (segment (start 143.002 102.87) (end 143.002 98.552) (width 0.25) (layer B.Cu) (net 14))
 (segment (start 143.002 98.552) (end 141.732 97.282) (width 0.25) (layer B.Cu) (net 14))
 (segment (start 141.732 97.282) (end 139.954 97.282) (width 0.25) (layer B.Cu) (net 14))
 (via (at 138.938 98.806) (size 0.8) (drill 0.4) (layers F.Cu B.Cu) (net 14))
 (segment (start 139.954 97.282) (end 138.938 98.298) (width 0.25) (layer B.Cu) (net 14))
 (segment (start 138.938 98.298) (end 138.938 98.806) (width 0.25) (layer B.Cu) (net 14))
 (segment (start 138.938 98.806) (end 138.938 100.584) (width 0.25) (layer F.Cu) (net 14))
 (segment (start 140.374 102.02) (end 142.994 102.02) (width 0.25) (layer F.Cu) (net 14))
 (segment (start 138.938 100.584) (end 140.374 102.02) (width 0.25) (layer F.Cu) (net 14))
 (segment (start 146.304 110.998) (end 144.018 110.998) (width 0.25) (layer B.Cu) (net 15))
 (segment (start 144.018 110.998) (end 139.446 106.426) (width 0.25) (layer B.Cu) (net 15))
 (via (at 139.446 103.124) (size 0.8) (drill 0.4) (layers F.Cu B.Cu) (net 15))
 (segment (start 139.446 106.426) (end 139.446 103.124) (width 0.25) (layer B.Cu) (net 15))
 (segment (start 142.898 103.124) (end 142.994 103.22) (width 0.25) (layer F.Cu) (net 15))
 (segment (start 139.446 103.124) (end 142.898 103.124) (width 0.25) (layer F.Cu) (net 15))
 (segment (start 146.304 113.538) (end 145.034 113.538) (width 0.25) (layer B.Cu) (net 16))
 (via (at 137.16 104.394) (size 0.8) (drill 0.4) (layers F.Cu B.Cu) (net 16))
 (segment (start 145.034 113.538) (end 137.16 105.664) (width 0.25) (layer B.Cu) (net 16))
 (segment (start 137.16 105.664) (end 137.16 104.394) (width 0.25) (layer B.Cu) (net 16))
 (segment (start 142.968 104.394) (end 142.994 104.42) (width 0.25) (layer F.Cu) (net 16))
 (segment (start 137.16 104.394) (end 142.968 104.394) (width 0.25) (layer F.Cu) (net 16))
 (segment (start 142.994 112.768) (end 142.994 105.62) (width 0.25) (layer F.Cu) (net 17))
 (segment (start 146.304 116.078) (end 142.994 112.768) (width 0.25) (layer F.Cu) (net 17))
 (segment (start 140.944 113.258) (end 140.944 106.67) (width 0.25) (layer F.Cu) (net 18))
 (segment (start 146.304 118.618) (end 140.944 113.258) (width 0.25) (layer F.Cu) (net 18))
 (segment (start 139.744 114.598) (end 146.304 121.158) (width 0.25) (layer F.Cu) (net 19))
 (segment (start 139.744 106.67) (end 139.744 114.598) (width 0.25) (layer F.Cu) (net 19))
 (segment (start 138.544 115.938) (end 138.544 106.67) (width 0.25) (layer F.Cu) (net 20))
 (segment (start 146.304 123.698) (end 138.544 115.938) (width 0.25) (layer F.Cu) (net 20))
 (segment (start 137.344 106.67) (end 137.344 118.548) (width 0.25) (layer F.Cu) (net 21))
 (segment (start 145.034 126.238) (end 146.304 126.238) (width 0.25) (layer F.Cu) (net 21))
 (segment (start 137.344 118.548) (end 145.034 126.238) (width 0.25) (layer F.Cu) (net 21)))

